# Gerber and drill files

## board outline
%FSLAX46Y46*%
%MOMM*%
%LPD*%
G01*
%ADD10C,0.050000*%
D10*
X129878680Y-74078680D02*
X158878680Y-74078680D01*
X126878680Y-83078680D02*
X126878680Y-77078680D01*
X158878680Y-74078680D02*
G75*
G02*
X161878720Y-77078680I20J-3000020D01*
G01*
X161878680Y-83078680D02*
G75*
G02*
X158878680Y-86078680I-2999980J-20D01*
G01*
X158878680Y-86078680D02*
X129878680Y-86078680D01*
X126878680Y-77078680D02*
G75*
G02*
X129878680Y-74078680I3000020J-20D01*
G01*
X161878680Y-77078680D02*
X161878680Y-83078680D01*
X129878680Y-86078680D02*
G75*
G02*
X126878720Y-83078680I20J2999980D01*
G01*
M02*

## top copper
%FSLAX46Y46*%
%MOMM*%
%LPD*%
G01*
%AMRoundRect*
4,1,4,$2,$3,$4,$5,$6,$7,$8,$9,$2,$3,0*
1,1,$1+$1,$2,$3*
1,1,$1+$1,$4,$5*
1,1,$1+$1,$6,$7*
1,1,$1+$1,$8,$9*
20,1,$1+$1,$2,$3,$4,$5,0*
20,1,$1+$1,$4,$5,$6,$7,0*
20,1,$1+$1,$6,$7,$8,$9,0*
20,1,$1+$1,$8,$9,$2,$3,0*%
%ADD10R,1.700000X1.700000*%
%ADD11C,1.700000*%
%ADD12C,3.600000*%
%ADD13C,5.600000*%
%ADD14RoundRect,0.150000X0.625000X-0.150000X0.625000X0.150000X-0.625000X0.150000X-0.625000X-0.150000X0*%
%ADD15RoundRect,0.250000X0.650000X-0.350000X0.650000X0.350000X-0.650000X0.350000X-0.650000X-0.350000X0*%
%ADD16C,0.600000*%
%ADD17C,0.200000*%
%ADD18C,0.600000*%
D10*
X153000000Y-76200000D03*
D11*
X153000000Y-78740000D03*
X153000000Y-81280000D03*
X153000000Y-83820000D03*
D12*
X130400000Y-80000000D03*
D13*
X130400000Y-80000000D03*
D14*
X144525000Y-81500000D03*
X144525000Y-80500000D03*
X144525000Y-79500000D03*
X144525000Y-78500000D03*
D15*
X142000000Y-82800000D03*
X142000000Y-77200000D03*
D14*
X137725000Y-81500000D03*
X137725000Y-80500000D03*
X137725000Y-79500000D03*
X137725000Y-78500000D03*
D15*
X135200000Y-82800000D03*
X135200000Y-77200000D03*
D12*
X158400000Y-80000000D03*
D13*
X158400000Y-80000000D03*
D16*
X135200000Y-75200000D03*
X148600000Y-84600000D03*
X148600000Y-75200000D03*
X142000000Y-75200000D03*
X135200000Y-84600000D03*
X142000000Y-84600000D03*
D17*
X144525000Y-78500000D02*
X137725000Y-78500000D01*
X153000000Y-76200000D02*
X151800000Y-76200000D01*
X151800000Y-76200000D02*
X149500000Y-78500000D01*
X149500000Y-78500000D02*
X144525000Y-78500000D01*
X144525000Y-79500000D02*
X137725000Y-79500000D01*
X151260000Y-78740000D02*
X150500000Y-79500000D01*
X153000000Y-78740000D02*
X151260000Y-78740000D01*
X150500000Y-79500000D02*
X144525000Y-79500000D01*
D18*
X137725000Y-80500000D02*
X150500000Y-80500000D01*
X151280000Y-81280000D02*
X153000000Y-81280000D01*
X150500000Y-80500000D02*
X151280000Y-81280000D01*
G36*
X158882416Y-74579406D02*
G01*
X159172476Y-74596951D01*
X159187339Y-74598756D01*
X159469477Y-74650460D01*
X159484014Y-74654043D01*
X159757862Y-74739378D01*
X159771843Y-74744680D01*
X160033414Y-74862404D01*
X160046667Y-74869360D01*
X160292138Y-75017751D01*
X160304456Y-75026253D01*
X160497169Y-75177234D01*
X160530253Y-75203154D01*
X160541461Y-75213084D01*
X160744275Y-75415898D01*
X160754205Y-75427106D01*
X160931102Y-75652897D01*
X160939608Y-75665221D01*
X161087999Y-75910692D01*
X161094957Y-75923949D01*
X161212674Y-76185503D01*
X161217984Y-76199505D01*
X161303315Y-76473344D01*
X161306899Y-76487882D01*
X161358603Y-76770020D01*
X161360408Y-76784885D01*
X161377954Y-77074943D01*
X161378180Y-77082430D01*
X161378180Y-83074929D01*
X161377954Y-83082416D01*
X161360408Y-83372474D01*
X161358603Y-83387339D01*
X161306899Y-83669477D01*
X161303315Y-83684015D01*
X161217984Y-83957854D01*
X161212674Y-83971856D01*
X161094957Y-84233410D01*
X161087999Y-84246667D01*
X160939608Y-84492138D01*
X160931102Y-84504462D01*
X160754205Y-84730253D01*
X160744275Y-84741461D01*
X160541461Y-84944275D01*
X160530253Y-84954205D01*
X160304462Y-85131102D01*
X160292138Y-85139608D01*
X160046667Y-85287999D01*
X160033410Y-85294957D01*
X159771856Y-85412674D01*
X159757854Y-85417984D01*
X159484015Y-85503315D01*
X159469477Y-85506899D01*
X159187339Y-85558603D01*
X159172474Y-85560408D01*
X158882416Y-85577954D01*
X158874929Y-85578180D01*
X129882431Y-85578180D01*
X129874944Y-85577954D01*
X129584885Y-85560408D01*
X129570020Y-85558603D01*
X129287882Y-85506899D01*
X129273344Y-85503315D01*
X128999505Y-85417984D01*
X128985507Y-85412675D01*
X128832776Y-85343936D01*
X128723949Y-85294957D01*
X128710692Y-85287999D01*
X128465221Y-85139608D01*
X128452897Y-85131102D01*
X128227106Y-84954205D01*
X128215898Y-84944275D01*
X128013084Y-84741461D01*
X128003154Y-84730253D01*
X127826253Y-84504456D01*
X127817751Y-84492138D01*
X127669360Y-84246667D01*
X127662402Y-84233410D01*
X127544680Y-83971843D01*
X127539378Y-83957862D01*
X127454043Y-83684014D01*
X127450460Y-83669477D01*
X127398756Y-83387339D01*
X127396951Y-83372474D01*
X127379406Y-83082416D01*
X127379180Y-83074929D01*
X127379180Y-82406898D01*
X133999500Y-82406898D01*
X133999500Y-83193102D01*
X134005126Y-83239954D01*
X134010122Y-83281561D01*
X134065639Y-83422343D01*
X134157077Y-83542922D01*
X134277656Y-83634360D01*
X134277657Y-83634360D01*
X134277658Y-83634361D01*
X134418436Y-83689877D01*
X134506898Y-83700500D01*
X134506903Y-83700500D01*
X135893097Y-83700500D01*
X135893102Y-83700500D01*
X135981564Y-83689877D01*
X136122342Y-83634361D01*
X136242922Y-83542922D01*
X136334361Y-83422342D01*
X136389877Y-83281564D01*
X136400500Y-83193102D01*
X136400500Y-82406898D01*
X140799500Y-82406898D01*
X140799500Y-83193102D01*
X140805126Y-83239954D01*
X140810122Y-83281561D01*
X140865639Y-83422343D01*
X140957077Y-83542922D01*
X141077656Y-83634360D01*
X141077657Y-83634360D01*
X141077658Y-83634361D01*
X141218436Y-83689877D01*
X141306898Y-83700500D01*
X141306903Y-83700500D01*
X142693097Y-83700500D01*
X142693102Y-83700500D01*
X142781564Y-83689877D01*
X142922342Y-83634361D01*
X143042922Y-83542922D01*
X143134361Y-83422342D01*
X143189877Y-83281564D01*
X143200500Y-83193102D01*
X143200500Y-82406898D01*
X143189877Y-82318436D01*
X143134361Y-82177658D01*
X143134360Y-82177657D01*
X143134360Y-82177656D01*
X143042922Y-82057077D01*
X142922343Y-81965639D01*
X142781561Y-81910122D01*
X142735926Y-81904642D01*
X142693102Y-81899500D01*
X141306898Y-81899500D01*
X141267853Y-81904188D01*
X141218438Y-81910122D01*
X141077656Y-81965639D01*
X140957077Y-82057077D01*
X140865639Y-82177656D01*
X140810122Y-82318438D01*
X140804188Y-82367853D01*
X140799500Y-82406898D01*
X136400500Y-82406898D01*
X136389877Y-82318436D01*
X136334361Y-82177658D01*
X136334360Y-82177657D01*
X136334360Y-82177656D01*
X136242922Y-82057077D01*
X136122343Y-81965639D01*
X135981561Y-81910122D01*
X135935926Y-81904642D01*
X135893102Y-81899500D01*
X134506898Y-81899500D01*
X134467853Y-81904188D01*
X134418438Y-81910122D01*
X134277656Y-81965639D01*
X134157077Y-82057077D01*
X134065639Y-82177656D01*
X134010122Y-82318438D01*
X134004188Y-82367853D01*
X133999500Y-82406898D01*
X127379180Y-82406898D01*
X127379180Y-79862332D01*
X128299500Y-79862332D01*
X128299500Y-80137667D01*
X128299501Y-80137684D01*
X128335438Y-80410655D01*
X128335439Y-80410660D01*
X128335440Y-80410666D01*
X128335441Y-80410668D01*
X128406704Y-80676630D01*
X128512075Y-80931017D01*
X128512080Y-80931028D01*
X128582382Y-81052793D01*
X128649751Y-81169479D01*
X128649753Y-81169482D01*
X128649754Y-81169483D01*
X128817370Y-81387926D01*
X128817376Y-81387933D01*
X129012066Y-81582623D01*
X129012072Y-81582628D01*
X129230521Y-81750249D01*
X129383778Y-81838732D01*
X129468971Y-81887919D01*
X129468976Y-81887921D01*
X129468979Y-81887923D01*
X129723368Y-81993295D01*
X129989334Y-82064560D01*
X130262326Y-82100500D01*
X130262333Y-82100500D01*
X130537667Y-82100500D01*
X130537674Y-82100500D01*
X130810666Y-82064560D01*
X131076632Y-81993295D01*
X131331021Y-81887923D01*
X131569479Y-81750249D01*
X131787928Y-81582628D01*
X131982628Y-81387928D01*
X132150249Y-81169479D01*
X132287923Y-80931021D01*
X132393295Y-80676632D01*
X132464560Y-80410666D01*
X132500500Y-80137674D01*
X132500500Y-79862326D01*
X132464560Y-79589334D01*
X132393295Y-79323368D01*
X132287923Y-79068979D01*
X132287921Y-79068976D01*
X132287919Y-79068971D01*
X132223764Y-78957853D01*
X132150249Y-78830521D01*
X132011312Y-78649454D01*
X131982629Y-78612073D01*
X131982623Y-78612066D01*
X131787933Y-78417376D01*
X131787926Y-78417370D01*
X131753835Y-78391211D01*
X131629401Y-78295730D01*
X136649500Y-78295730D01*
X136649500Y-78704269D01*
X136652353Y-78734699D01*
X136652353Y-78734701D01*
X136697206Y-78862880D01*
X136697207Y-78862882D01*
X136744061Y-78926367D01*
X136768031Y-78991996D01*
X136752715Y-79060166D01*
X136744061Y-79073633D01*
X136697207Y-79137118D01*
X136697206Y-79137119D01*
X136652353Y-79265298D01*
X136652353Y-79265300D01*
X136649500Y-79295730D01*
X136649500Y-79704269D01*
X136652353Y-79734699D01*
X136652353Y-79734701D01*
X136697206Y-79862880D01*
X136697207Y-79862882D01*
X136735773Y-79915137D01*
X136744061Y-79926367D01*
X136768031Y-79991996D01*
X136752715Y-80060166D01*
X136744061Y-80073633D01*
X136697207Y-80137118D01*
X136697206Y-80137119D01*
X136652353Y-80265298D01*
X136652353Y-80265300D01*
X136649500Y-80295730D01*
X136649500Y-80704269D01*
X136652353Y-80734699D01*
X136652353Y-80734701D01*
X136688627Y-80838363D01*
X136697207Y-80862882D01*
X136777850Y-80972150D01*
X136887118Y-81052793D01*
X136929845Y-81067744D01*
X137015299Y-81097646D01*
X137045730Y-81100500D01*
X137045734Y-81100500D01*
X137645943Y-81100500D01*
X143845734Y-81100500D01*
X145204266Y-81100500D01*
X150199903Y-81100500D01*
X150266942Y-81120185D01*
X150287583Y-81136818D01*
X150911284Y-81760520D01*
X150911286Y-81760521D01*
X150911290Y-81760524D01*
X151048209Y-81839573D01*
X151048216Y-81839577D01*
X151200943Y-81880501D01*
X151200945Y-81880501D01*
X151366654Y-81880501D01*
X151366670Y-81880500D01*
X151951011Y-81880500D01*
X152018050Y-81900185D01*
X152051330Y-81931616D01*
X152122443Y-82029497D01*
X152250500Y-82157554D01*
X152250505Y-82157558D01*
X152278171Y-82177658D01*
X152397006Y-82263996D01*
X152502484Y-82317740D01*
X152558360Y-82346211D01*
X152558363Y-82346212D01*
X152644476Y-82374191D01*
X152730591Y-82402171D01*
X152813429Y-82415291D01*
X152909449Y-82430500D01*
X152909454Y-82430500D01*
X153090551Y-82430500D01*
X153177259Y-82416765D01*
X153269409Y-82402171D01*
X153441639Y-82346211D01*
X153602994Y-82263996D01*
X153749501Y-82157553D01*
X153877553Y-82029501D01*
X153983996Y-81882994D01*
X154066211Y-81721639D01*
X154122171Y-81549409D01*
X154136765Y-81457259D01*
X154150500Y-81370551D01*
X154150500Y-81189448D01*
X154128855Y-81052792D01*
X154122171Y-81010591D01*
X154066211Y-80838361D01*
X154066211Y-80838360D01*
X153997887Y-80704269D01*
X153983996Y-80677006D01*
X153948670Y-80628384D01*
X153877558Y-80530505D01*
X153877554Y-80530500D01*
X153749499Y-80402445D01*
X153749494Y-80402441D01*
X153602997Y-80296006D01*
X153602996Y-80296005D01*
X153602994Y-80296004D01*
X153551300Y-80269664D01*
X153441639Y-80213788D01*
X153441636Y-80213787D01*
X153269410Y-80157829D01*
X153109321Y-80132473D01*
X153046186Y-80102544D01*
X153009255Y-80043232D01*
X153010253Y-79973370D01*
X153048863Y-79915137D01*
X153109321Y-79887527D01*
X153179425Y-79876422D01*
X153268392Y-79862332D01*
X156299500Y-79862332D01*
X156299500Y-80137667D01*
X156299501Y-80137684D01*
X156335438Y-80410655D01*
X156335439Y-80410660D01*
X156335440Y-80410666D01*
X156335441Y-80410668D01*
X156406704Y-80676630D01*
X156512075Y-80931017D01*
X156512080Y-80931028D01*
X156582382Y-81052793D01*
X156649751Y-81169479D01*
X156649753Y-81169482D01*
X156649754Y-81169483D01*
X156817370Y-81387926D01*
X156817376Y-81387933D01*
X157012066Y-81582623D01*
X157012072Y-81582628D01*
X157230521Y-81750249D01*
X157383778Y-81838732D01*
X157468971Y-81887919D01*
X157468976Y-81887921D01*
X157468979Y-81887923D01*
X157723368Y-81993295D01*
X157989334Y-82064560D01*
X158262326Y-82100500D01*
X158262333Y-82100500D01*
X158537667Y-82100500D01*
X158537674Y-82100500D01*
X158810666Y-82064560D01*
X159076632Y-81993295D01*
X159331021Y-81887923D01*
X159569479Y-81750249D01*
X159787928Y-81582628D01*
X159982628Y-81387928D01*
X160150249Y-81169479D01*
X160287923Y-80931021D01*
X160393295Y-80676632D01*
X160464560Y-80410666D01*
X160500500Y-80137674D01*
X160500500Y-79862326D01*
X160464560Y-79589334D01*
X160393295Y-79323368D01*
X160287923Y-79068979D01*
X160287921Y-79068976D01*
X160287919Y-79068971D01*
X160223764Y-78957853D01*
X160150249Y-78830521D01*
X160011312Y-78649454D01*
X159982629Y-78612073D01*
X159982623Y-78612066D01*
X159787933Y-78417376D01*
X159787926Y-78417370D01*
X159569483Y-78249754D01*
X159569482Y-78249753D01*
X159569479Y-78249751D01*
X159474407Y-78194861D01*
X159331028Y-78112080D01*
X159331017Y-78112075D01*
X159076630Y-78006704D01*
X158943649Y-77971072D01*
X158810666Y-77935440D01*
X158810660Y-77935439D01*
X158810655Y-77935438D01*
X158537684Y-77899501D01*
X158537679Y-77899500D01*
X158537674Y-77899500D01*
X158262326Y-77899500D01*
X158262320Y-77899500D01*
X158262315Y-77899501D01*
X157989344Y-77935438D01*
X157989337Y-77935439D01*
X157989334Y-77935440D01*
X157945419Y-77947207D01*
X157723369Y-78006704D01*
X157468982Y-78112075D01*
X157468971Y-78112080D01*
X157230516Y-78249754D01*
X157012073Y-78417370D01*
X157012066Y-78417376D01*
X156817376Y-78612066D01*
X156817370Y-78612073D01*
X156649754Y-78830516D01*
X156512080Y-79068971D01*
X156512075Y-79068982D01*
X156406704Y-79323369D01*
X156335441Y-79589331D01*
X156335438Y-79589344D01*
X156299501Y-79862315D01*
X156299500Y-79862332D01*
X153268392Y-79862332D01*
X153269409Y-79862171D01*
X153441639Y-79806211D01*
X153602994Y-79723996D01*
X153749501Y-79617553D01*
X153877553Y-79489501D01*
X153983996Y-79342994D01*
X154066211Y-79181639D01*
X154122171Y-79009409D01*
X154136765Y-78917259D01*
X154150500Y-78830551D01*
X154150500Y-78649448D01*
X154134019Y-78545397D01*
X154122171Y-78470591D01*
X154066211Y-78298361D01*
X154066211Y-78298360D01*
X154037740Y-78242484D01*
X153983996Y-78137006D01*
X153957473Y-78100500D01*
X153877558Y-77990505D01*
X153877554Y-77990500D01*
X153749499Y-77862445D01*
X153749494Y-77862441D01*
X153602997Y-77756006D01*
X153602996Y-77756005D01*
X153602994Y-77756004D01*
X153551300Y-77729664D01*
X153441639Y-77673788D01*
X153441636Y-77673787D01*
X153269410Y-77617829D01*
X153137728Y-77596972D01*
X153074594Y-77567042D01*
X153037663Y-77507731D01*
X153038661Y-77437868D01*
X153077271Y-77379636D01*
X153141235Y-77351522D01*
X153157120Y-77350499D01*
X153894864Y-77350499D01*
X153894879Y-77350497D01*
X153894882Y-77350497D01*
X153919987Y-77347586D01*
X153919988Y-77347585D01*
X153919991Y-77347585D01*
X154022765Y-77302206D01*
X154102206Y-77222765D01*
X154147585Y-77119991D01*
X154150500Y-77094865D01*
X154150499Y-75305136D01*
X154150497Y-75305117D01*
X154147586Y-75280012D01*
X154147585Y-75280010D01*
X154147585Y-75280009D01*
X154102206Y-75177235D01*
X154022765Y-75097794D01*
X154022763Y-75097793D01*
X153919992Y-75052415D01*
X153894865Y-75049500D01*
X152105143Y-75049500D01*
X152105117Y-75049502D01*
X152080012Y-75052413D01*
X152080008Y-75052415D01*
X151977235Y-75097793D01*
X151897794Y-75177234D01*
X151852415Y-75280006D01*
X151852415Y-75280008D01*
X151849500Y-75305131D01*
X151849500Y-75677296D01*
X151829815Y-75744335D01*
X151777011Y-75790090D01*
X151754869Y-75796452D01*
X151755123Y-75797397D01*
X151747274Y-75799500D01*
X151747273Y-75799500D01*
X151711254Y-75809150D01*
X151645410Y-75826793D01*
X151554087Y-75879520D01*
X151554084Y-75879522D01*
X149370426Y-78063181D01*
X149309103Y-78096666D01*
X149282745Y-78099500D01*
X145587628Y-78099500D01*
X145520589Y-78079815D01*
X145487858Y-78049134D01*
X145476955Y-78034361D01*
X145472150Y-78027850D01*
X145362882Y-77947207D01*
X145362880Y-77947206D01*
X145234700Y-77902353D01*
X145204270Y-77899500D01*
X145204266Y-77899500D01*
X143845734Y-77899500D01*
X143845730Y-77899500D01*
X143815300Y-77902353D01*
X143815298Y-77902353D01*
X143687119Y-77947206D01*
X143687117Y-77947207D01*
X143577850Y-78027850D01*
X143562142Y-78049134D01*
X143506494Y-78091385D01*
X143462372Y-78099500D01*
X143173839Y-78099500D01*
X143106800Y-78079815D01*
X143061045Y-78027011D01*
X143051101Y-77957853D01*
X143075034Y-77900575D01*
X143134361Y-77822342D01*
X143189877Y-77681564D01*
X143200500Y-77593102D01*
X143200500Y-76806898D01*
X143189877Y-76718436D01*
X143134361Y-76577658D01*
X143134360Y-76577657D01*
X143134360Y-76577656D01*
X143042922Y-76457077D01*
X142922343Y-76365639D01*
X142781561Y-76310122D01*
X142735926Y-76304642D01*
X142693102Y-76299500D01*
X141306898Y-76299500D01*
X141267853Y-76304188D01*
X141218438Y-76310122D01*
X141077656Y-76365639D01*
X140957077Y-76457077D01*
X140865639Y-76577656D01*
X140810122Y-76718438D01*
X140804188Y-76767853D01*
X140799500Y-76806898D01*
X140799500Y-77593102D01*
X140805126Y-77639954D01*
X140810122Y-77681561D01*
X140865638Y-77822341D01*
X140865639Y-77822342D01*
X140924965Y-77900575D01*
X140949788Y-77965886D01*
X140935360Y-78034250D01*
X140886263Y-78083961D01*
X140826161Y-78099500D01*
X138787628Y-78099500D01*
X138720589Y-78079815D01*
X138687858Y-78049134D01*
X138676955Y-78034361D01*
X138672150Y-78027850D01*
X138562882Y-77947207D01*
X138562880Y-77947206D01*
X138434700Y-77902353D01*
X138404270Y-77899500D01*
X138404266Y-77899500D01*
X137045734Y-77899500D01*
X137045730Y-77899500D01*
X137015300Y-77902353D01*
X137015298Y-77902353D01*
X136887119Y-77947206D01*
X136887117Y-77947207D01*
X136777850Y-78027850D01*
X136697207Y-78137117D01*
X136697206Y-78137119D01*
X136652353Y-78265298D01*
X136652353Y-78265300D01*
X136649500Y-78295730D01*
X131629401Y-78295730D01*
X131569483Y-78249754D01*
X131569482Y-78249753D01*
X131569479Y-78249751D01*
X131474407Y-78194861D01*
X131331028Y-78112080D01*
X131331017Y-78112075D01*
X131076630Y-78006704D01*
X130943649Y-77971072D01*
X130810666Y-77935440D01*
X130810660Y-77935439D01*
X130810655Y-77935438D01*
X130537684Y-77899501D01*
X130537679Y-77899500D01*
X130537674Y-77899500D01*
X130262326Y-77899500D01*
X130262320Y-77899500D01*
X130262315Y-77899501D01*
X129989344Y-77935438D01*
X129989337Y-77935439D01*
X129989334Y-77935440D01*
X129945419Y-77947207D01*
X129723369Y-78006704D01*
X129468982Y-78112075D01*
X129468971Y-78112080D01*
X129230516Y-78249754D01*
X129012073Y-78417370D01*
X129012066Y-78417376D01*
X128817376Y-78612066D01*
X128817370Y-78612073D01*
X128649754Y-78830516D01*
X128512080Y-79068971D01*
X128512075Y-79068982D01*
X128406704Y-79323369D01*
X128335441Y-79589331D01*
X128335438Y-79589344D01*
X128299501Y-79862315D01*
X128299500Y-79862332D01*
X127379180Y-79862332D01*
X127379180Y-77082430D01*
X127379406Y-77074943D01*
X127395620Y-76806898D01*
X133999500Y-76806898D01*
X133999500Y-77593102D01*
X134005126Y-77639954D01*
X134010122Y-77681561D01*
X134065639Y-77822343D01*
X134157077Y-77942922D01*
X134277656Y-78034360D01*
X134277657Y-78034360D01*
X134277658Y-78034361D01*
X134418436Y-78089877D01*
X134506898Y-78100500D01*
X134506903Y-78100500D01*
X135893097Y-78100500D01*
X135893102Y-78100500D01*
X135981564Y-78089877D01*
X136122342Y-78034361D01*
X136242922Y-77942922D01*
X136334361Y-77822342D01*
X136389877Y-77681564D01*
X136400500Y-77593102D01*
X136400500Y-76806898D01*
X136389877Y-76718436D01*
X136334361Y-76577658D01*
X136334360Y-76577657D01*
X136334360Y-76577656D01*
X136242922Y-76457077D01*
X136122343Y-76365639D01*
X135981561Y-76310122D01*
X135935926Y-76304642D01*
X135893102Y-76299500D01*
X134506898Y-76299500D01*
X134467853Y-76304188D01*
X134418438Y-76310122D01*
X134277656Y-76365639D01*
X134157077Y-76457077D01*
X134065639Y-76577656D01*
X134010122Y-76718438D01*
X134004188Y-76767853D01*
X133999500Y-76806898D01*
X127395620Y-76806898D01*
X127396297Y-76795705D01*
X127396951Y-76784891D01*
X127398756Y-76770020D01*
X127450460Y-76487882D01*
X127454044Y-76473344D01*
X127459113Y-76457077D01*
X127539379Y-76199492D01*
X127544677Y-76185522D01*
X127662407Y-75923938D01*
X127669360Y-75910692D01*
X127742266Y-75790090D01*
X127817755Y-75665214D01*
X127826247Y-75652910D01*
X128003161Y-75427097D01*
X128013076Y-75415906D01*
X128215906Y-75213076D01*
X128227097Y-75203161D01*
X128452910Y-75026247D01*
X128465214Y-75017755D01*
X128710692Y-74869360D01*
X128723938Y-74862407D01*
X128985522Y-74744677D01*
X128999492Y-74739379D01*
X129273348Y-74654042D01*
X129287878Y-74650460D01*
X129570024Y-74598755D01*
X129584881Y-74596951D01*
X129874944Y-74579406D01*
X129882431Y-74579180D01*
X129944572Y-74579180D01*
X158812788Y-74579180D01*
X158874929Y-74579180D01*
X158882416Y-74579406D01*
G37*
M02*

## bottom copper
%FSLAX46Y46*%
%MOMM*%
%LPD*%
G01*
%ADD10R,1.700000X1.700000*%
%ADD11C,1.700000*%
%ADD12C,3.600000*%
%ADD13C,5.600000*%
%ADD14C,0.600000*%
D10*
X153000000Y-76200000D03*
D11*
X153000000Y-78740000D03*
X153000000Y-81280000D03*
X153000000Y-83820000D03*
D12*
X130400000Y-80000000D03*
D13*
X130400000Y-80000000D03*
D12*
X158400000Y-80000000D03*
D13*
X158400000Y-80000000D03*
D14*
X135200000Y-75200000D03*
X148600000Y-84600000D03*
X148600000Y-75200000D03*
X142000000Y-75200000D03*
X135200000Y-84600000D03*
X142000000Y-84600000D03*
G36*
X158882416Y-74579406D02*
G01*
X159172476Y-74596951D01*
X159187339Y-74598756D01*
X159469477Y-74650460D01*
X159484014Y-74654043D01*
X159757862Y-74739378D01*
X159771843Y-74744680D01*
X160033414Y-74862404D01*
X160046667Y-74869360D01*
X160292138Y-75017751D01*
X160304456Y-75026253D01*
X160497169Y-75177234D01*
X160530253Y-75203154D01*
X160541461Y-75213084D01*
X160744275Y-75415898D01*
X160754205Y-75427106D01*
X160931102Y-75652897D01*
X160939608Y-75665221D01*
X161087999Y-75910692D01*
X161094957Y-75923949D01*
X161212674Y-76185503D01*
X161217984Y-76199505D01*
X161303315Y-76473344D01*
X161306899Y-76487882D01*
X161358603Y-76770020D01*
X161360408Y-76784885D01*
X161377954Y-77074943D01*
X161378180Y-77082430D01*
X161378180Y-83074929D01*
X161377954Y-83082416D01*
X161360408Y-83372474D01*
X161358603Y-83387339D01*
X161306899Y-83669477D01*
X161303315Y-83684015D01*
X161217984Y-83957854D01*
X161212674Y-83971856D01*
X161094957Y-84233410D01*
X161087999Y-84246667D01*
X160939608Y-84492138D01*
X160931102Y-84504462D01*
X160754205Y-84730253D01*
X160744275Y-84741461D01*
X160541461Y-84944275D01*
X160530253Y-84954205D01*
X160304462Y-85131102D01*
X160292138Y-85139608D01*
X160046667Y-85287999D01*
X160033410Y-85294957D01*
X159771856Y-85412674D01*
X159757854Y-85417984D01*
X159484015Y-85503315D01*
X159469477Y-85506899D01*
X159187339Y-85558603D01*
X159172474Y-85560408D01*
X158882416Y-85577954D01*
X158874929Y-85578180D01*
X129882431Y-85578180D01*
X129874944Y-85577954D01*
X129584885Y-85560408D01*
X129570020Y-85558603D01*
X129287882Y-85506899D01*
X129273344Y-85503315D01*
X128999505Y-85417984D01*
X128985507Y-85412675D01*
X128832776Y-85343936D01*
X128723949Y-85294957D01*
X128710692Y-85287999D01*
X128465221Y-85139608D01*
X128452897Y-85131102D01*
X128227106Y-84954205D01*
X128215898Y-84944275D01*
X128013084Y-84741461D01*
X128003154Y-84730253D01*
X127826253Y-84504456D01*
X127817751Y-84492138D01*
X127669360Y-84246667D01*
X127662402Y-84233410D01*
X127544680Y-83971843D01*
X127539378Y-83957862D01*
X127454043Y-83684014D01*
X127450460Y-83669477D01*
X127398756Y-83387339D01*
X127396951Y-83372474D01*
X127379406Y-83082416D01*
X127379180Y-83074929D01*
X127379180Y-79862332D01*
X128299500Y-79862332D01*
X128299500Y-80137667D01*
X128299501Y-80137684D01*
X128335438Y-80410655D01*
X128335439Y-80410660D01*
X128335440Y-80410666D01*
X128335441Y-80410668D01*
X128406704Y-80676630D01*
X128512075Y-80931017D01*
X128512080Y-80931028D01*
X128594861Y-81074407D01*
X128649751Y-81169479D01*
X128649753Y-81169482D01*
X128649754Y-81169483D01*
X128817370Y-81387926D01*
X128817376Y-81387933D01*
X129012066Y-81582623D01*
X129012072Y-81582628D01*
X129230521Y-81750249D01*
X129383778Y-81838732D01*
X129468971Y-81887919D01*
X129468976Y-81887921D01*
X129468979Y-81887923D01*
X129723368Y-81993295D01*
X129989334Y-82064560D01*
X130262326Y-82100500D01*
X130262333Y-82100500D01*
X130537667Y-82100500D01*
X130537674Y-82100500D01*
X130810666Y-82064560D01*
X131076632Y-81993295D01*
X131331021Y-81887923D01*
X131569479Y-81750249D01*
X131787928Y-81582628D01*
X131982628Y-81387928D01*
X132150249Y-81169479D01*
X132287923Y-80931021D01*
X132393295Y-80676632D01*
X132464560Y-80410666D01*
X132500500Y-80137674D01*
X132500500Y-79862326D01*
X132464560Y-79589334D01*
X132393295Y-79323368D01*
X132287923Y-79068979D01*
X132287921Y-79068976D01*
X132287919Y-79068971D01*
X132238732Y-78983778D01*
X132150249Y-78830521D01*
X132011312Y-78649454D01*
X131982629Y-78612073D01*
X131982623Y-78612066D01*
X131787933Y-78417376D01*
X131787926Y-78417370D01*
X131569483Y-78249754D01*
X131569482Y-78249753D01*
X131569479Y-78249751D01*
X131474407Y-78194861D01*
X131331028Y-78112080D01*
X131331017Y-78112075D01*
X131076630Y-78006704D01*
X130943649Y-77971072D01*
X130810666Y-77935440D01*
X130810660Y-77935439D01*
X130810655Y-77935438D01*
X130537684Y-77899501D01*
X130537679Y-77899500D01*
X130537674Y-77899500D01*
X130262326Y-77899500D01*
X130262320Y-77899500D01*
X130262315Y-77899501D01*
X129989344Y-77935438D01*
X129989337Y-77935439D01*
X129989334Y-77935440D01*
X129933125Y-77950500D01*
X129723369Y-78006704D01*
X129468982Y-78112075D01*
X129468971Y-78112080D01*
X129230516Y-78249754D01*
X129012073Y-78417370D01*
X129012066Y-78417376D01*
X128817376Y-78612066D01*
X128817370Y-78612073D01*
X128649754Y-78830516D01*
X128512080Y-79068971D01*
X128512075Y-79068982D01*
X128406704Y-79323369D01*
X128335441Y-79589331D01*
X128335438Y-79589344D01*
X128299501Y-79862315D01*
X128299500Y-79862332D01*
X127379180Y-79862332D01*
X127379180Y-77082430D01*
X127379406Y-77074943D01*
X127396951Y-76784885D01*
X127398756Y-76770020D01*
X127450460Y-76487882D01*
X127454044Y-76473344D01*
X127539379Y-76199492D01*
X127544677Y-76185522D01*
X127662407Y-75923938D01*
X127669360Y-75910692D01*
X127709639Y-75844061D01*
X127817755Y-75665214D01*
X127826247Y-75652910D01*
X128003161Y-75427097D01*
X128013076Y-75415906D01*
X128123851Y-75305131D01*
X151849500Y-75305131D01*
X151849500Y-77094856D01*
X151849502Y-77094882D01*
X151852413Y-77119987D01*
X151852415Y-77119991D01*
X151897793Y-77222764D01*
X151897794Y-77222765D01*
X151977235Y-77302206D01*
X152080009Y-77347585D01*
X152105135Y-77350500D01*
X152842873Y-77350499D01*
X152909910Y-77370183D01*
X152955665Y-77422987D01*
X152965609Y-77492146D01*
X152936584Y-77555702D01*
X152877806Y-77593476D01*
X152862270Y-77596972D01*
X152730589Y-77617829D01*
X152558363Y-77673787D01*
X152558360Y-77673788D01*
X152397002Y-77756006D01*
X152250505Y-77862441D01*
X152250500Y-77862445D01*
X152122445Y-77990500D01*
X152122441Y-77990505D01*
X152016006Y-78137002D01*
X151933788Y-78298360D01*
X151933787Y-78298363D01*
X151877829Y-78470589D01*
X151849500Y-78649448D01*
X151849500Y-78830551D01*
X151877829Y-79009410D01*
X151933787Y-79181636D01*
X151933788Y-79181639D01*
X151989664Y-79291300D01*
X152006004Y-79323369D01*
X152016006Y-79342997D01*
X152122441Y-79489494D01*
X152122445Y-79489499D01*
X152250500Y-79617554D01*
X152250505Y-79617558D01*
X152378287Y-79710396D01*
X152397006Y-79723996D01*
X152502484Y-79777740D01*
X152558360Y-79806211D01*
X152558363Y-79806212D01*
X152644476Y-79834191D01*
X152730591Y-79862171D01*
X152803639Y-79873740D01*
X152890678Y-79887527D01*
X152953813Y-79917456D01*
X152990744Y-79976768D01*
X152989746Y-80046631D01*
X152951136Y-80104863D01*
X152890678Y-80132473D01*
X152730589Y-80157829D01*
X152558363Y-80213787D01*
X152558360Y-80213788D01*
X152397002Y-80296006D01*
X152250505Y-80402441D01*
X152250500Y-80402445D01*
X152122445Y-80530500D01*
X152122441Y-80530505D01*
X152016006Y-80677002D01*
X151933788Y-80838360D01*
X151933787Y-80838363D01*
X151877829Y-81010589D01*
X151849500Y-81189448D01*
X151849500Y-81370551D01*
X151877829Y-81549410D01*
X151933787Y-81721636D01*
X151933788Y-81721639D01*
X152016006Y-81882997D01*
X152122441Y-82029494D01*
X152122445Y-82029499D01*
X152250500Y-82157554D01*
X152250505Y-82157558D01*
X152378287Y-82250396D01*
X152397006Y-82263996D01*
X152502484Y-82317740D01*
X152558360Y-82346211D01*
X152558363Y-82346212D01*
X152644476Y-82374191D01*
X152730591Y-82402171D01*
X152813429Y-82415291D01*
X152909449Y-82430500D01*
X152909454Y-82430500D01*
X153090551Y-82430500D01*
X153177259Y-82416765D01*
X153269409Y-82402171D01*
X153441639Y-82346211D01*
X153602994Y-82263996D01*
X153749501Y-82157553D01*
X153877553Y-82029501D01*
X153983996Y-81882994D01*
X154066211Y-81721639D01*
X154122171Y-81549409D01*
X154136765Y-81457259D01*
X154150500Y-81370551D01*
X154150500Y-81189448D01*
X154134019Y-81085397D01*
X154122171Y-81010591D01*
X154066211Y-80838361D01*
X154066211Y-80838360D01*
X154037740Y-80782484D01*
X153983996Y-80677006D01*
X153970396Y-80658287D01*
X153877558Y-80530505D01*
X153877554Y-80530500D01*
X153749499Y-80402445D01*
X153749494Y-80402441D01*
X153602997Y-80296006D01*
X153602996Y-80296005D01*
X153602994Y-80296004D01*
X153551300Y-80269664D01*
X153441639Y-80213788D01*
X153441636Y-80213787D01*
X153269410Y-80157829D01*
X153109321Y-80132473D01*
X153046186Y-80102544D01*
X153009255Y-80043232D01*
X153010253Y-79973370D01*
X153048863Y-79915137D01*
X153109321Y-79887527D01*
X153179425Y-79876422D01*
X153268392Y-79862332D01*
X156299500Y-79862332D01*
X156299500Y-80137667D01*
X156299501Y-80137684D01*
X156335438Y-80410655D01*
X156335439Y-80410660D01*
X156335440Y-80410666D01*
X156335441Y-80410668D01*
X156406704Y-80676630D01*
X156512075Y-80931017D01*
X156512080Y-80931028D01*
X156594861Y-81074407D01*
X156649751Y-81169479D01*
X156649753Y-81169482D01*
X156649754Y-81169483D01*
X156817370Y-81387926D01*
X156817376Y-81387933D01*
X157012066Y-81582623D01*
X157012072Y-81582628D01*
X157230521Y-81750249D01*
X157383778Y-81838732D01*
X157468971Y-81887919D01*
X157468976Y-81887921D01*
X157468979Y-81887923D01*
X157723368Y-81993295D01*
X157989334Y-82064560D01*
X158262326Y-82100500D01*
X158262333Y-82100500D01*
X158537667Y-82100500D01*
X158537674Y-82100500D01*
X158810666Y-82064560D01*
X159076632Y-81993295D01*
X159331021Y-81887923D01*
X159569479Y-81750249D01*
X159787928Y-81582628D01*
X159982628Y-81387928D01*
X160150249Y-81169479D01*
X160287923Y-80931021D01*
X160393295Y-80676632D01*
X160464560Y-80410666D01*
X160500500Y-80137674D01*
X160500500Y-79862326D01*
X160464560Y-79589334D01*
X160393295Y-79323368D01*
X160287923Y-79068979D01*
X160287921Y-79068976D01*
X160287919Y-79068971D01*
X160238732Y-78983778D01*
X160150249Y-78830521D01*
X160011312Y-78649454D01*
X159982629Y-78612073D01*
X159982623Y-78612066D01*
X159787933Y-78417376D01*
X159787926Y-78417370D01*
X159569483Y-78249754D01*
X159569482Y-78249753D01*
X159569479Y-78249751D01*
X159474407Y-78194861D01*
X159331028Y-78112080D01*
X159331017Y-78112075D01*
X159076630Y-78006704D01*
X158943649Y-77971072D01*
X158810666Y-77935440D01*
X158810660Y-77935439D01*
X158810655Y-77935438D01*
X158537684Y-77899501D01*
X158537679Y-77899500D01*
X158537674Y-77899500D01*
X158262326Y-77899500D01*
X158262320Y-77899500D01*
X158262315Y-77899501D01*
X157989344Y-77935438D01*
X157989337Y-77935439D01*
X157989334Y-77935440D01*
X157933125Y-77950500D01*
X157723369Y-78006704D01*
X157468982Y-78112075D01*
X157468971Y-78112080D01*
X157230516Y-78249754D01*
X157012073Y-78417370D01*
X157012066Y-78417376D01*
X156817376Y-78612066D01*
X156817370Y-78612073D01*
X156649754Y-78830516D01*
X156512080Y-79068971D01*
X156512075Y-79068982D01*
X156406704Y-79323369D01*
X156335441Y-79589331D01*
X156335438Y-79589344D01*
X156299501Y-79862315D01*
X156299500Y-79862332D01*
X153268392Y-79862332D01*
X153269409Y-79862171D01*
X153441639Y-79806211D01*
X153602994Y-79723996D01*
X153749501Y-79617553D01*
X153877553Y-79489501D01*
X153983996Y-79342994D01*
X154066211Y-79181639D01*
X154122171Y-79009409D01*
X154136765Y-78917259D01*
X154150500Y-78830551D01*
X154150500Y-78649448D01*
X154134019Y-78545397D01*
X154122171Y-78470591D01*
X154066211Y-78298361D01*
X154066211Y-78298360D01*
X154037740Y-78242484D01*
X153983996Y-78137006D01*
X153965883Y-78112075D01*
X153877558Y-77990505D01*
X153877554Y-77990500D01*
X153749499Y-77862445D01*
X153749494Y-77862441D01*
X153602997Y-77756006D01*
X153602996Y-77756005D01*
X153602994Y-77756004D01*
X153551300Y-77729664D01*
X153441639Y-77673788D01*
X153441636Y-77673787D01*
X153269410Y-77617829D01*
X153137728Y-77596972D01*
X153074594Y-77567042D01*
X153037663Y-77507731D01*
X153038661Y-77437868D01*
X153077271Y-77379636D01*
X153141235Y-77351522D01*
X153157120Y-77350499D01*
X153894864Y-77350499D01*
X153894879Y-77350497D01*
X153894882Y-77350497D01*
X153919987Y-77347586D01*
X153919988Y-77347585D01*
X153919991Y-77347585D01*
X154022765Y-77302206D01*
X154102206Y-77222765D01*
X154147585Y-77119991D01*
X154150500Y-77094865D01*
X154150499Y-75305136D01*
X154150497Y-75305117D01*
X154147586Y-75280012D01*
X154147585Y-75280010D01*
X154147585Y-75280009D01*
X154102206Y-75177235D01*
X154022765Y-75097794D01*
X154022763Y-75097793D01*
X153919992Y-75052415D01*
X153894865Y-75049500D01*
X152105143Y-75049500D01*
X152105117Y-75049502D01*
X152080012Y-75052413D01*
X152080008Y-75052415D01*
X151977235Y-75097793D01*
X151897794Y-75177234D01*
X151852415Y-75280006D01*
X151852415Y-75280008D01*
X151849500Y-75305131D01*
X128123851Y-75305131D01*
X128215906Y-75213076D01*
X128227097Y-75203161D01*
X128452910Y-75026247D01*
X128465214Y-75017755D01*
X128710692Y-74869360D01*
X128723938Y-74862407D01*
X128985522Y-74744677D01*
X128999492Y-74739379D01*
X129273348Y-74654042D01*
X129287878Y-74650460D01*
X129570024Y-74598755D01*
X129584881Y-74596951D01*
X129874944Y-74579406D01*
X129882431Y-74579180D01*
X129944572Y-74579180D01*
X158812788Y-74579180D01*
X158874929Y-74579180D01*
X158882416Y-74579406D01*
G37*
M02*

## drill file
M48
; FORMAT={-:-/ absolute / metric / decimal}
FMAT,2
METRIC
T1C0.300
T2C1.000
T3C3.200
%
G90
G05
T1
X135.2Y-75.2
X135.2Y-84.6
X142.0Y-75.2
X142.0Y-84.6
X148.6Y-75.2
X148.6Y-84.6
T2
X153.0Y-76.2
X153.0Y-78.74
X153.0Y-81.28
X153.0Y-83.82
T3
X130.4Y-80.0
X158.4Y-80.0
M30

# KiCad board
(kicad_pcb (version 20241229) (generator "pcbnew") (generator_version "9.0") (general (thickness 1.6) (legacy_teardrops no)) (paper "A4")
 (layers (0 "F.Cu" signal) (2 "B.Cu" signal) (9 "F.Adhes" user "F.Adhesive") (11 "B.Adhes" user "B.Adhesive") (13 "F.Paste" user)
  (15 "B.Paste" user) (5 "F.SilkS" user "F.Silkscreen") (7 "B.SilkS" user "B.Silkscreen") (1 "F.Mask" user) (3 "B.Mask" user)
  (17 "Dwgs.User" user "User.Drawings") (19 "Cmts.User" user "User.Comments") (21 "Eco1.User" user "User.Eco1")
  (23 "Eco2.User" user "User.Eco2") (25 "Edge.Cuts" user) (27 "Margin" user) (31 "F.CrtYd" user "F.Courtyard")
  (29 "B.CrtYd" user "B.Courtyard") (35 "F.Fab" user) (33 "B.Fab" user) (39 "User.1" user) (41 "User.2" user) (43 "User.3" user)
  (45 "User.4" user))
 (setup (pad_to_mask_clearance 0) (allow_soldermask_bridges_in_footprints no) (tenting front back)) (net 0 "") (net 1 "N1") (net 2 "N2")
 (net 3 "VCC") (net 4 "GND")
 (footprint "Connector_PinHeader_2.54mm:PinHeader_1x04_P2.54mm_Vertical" (layer "F.Cu") (at 153 76.2)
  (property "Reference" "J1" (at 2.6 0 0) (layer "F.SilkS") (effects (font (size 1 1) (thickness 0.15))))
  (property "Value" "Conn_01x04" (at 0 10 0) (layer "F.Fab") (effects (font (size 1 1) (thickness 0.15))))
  (pad "1" thru_hole rect (at 0 0) (size 1.7 1.7) (drill 1) (layers "*.Cu" "*.Mask") (remove_unused_layers no) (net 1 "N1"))
  (pad "2" thru_hole circle (at 0 2.54) (size 1.7 1.7) (drill 1) (layers "*.Cu" "*.Mask") (remove_unused_layers no) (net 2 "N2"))
  (pad "3" thru_hole circle (at 0 5.08) (size 1.7 1.7) (drill 1) (layers "*.Cu" "*.Mask") (remove_unused_layers no) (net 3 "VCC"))
  (pad "4" thru_hole circle (at 0 7.62) (size 1.7 1.7) (drill 1) (layers "*.Cu" "*.Mask") (remove_unused_layers no) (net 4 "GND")))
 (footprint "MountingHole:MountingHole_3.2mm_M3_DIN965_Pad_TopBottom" (layer "F.Cu") (at 130.4 80)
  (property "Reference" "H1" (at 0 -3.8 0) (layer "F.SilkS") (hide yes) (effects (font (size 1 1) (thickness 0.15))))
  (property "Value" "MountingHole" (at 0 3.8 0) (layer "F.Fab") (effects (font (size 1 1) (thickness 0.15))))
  (pad "1" thru_hole circle (at 0 0) (size 3.6 3.6) (drill 3.2) (layers "*.Cu" "*.Mask") (remove_unused_layers no))
  (pad "1" connect circle (at 0 0) (size 5.6 5.6) (layers "F.Cu" "F.Mask") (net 4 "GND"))
  (pad "1" connect circle (at 0 0) (size 5.6 5.6) (layers "B.Cu" "B.Mask") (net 4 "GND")))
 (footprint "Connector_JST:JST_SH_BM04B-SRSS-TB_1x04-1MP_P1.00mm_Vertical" (layer "F.Cu") (at 143.2 80 90)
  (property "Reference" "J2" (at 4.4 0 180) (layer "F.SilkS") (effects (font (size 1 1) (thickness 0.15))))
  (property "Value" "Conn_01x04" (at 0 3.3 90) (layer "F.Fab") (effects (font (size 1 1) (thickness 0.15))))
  (pad "1" smd roundrect (at -1.5 1.325 90) (size 0.6 1.55) (layers "F.Cu" "F.Mask" "F.Paste") (roundrect_rratio 0.25) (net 4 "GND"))
  (pad "2" smd roundrect (at -0.5 1.325 90) (size 0.6 1.55) (layers "F.Cu" "F.Mask" "F.Paste") (roundrect_rratio 0.25) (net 3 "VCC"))
  (pad "3" smd roundrect (at 0.5 1.325 90) (size 0.6 1.55) (layers "F.Cu" "F.Mask" "F.Paste") (roundrect_rratio 0.25) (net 2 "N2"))
  (pad "4" smd roundrect (at 1.5 1.325 90) (size 0.6 1.55) (layers "F.Cu" "F.Mask" "F.Paste") (roundrect_rratio 0.25) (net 1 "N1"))
  (pad "MP" smd roundrect (at -2.8 -1.2 90) (size 1.2 1.8) (layers "F.Cu" "F.Mask" "F.Paste") (roundrect_rratio 0.208333))
  (pad "MP" smd roundrect (at 2.8 -1.2 90) (size 1.2 1.8) (layers "F.Cu" "F.Mask" "F.Paste") (roundrect_rratio 0.208333)))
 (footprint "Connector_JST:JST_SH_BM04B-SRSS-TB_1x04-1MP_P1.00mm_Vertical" (layer "F.Cu") (at 136.4 80 90)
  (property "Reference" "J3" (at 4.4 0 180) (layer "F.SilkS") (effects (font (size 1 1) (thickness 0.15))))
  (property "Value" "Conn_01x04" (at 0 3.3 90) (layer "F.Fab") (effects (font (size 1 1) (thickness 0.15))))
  (pad "1" smd roundrect (at -1.5 1.325 90) (size 0.6 1.55) (layers "F.Cu" "F.Mask" "F.Paste") (roundrect_rratio 0.25) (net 4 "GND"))
  (pad "2" smd roundrect (at -0.5 1.325 90) (size 0.6 1.55) (layers "F.Cu" "F.Mask" "F.Paste") (roundrect_rratio 0.25) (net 3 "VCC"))
  (pad "3" smd roundrect (at 0.5 1.325 90) (size 0.6 1.55) (layers "F.Cu" "F.Mask" "F.Paste") (roundrect_rratio 0.25) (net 2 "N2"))
  (pad "4" smd roundrect (at 1.5 1.325 90) (size 0.6 1.55) (layers "F.Cu" "F.Mask" "F.Paste") (roundrect_rratio 0.25) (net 1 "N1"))
  (pad "MP" smd roundrect (at -2.8 -1.2 90) (size 1.2 1.8) (layers "F.Cu" "F.Mask" "F.Paste") (roundrect_rratio 0.208333))
  (pad "MP" smd roundrect (at 2.8 -1.2 90) (size 1.2 1.8) (layers "F.Cu" "F.Mask" "F.Paste") (roundrect_rratio 0.208333)))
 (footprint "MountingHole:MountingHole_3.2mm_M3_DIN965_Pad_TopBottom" (layer "F.Cu") (at 158.4 80)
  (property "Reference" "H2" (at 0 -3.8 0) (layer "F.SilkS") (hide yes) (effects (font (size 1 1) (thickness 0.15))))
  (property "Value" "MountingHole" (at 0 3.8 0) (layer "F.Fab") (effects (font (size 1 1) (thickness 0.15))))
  (pad "1" thru_hole circle (at 0 0) (size 3.6 3.6) (drill 3.2) (layers "*.Cu" "*.Mask") (remove_unused_layers no))
  (pad "1" connect circle (at 0 0) (size 5.6 5.6) (layers "F.Cu" "F.Mask") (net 4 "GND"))
  (pad "1" connect circle (at 0 0) (size 5.6 5.6) (layers "B.Cu" "B.Mask") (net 4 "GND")))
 (gr_line (start 129.87868 74.07868) (end 158.87868 74.07868) (stroke (width 0.05) (type default)) (layer "Edge.Cuts"))
 (gr_line (start 126.87868 83.07868) (end 126.87868 77.07868) (stroke (width 0.05) (type default)) (layer "Edge.Cuts"))
 (gr_arc (start 158.87868 74.07868) (mid 161 74.95736) (end 161.87868 77.07868) (stroke (width 0.05) (type solid)) (layer "Edge.Cuts"))
 (gr_arc (start 161.87868 83.07868) (mid 161 85.2) (end 158.87868 86.07868) (stroke (width 0.05) (type solid)) (layer "Edge.Cuts"))
 (gr_line (start 158.87868 86.07868) (end 129.87868 86.07868) (stroke (width 0.05) (type default)) (layer "Edge.Cuts"))
 (gr_arc (start 126.87868 77.07868) (mid 127.75736 74.95736) (end 129.87868 74.07868) (stroke (width 0.05) (type solid)) (layer "Edge.Cuts"))
 (gr_line (start 161.87868 77.07868) (end 161.87868 83.07868) (stroke (width 0.05) (type default)) (layer "Edge.Cuts"))
 (gr_arc (start 129.87868 86.07868) (mid 127.75736 85.2) (end 126.87868 83.07868) (stroke (width 0.05) (type solid)) (layer "Edge.Cuts"))
 (via (at 135.2 75.2) (size 0.6) (drill 0.3) (layers "F.Cu" "B.Cu") (free yes) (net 4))
 (via (at 148.6 84.6) (size 0.6) (drill 0.3) (layers "F.Cu" "B.Cu") (free yes) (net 4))
 (via (at 148.6 75.2) (size 0.6) (drill 0.3) (layers "F.Cu" "B.Cu") (free yes) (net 4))
 (via (at 142 75.2) (size 0.6) (drill 0.3) (layers "F.Cu" "B.Cu") (free yes) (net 4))
 (via (at 135.2 84.6) (size 0.6) (drill 0.3) (layers "F.Cu" "B.Cu") (free yes) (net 4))
 (via (at 142 84.6) (size 0.6) (drill 0.3) (layers "F.Cu" "B.Cu") (free yes) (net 4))
 (segment (start 144.525 78.5) (end 137.725 78.5) (width 0.2) (layer "F.Cu") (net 1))
 (segment (start 153 76.2) (end 151.8 76.2) (width 0.2) (layer "F.Cu") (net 1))
 (segment (start 151.8 76.2) (end 149.5 78.5) (width 0.2) (layer "F.Cu") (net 1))
 (segment (start 149.5 78.5) (end 144.525 78.5) (width 0.2) (layer "F.Cu") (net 1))
 (segment (start 144.525 79.5) (end 137.725 79.5) (width 0.2) (layer "F.Cu") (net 2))
 (segment (start 151.26 78.74) (end 150.5 79.5) (width 0.2) (layer "F.Cu") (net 2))
 (segment (start 153 78.74) (end 151.26 78.74) (width 0.2) (layer "F.Cu") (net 2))
 (segment (start 150.5 79.5) (end 144.525 79.5) (width 0.2) (layer "F.Cu") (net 2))
 (segment (start 137.725 80.5) (end 150.5 80.5) (width 0.6) (layer "F.Cu") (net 3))
 (segment (start 151.28 81.28) (end 153 81.28) (width 0.6) (layer "F.Cu") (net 3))
 (segment (start 150.5 80.5) (end 151.28 81.28) (width 0.6) (layer "F.Cu") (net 3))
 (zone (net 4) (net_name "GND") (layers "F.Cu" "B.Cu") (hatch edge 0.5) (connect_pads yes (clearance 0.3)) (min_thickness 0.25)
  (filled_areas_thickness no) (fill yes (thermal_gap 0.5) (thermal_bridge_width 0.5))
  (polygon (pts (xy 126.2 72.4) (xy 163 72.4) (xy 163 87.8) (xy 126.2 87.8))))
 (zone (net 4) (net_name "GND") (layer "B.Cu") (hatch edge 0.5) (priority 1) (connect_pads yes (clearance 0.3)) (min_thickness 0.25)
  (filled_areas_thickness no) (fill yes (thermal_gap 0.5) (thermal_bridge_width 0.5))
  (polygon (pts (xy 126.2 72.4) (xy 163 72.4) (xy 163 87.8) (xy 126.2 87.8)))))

